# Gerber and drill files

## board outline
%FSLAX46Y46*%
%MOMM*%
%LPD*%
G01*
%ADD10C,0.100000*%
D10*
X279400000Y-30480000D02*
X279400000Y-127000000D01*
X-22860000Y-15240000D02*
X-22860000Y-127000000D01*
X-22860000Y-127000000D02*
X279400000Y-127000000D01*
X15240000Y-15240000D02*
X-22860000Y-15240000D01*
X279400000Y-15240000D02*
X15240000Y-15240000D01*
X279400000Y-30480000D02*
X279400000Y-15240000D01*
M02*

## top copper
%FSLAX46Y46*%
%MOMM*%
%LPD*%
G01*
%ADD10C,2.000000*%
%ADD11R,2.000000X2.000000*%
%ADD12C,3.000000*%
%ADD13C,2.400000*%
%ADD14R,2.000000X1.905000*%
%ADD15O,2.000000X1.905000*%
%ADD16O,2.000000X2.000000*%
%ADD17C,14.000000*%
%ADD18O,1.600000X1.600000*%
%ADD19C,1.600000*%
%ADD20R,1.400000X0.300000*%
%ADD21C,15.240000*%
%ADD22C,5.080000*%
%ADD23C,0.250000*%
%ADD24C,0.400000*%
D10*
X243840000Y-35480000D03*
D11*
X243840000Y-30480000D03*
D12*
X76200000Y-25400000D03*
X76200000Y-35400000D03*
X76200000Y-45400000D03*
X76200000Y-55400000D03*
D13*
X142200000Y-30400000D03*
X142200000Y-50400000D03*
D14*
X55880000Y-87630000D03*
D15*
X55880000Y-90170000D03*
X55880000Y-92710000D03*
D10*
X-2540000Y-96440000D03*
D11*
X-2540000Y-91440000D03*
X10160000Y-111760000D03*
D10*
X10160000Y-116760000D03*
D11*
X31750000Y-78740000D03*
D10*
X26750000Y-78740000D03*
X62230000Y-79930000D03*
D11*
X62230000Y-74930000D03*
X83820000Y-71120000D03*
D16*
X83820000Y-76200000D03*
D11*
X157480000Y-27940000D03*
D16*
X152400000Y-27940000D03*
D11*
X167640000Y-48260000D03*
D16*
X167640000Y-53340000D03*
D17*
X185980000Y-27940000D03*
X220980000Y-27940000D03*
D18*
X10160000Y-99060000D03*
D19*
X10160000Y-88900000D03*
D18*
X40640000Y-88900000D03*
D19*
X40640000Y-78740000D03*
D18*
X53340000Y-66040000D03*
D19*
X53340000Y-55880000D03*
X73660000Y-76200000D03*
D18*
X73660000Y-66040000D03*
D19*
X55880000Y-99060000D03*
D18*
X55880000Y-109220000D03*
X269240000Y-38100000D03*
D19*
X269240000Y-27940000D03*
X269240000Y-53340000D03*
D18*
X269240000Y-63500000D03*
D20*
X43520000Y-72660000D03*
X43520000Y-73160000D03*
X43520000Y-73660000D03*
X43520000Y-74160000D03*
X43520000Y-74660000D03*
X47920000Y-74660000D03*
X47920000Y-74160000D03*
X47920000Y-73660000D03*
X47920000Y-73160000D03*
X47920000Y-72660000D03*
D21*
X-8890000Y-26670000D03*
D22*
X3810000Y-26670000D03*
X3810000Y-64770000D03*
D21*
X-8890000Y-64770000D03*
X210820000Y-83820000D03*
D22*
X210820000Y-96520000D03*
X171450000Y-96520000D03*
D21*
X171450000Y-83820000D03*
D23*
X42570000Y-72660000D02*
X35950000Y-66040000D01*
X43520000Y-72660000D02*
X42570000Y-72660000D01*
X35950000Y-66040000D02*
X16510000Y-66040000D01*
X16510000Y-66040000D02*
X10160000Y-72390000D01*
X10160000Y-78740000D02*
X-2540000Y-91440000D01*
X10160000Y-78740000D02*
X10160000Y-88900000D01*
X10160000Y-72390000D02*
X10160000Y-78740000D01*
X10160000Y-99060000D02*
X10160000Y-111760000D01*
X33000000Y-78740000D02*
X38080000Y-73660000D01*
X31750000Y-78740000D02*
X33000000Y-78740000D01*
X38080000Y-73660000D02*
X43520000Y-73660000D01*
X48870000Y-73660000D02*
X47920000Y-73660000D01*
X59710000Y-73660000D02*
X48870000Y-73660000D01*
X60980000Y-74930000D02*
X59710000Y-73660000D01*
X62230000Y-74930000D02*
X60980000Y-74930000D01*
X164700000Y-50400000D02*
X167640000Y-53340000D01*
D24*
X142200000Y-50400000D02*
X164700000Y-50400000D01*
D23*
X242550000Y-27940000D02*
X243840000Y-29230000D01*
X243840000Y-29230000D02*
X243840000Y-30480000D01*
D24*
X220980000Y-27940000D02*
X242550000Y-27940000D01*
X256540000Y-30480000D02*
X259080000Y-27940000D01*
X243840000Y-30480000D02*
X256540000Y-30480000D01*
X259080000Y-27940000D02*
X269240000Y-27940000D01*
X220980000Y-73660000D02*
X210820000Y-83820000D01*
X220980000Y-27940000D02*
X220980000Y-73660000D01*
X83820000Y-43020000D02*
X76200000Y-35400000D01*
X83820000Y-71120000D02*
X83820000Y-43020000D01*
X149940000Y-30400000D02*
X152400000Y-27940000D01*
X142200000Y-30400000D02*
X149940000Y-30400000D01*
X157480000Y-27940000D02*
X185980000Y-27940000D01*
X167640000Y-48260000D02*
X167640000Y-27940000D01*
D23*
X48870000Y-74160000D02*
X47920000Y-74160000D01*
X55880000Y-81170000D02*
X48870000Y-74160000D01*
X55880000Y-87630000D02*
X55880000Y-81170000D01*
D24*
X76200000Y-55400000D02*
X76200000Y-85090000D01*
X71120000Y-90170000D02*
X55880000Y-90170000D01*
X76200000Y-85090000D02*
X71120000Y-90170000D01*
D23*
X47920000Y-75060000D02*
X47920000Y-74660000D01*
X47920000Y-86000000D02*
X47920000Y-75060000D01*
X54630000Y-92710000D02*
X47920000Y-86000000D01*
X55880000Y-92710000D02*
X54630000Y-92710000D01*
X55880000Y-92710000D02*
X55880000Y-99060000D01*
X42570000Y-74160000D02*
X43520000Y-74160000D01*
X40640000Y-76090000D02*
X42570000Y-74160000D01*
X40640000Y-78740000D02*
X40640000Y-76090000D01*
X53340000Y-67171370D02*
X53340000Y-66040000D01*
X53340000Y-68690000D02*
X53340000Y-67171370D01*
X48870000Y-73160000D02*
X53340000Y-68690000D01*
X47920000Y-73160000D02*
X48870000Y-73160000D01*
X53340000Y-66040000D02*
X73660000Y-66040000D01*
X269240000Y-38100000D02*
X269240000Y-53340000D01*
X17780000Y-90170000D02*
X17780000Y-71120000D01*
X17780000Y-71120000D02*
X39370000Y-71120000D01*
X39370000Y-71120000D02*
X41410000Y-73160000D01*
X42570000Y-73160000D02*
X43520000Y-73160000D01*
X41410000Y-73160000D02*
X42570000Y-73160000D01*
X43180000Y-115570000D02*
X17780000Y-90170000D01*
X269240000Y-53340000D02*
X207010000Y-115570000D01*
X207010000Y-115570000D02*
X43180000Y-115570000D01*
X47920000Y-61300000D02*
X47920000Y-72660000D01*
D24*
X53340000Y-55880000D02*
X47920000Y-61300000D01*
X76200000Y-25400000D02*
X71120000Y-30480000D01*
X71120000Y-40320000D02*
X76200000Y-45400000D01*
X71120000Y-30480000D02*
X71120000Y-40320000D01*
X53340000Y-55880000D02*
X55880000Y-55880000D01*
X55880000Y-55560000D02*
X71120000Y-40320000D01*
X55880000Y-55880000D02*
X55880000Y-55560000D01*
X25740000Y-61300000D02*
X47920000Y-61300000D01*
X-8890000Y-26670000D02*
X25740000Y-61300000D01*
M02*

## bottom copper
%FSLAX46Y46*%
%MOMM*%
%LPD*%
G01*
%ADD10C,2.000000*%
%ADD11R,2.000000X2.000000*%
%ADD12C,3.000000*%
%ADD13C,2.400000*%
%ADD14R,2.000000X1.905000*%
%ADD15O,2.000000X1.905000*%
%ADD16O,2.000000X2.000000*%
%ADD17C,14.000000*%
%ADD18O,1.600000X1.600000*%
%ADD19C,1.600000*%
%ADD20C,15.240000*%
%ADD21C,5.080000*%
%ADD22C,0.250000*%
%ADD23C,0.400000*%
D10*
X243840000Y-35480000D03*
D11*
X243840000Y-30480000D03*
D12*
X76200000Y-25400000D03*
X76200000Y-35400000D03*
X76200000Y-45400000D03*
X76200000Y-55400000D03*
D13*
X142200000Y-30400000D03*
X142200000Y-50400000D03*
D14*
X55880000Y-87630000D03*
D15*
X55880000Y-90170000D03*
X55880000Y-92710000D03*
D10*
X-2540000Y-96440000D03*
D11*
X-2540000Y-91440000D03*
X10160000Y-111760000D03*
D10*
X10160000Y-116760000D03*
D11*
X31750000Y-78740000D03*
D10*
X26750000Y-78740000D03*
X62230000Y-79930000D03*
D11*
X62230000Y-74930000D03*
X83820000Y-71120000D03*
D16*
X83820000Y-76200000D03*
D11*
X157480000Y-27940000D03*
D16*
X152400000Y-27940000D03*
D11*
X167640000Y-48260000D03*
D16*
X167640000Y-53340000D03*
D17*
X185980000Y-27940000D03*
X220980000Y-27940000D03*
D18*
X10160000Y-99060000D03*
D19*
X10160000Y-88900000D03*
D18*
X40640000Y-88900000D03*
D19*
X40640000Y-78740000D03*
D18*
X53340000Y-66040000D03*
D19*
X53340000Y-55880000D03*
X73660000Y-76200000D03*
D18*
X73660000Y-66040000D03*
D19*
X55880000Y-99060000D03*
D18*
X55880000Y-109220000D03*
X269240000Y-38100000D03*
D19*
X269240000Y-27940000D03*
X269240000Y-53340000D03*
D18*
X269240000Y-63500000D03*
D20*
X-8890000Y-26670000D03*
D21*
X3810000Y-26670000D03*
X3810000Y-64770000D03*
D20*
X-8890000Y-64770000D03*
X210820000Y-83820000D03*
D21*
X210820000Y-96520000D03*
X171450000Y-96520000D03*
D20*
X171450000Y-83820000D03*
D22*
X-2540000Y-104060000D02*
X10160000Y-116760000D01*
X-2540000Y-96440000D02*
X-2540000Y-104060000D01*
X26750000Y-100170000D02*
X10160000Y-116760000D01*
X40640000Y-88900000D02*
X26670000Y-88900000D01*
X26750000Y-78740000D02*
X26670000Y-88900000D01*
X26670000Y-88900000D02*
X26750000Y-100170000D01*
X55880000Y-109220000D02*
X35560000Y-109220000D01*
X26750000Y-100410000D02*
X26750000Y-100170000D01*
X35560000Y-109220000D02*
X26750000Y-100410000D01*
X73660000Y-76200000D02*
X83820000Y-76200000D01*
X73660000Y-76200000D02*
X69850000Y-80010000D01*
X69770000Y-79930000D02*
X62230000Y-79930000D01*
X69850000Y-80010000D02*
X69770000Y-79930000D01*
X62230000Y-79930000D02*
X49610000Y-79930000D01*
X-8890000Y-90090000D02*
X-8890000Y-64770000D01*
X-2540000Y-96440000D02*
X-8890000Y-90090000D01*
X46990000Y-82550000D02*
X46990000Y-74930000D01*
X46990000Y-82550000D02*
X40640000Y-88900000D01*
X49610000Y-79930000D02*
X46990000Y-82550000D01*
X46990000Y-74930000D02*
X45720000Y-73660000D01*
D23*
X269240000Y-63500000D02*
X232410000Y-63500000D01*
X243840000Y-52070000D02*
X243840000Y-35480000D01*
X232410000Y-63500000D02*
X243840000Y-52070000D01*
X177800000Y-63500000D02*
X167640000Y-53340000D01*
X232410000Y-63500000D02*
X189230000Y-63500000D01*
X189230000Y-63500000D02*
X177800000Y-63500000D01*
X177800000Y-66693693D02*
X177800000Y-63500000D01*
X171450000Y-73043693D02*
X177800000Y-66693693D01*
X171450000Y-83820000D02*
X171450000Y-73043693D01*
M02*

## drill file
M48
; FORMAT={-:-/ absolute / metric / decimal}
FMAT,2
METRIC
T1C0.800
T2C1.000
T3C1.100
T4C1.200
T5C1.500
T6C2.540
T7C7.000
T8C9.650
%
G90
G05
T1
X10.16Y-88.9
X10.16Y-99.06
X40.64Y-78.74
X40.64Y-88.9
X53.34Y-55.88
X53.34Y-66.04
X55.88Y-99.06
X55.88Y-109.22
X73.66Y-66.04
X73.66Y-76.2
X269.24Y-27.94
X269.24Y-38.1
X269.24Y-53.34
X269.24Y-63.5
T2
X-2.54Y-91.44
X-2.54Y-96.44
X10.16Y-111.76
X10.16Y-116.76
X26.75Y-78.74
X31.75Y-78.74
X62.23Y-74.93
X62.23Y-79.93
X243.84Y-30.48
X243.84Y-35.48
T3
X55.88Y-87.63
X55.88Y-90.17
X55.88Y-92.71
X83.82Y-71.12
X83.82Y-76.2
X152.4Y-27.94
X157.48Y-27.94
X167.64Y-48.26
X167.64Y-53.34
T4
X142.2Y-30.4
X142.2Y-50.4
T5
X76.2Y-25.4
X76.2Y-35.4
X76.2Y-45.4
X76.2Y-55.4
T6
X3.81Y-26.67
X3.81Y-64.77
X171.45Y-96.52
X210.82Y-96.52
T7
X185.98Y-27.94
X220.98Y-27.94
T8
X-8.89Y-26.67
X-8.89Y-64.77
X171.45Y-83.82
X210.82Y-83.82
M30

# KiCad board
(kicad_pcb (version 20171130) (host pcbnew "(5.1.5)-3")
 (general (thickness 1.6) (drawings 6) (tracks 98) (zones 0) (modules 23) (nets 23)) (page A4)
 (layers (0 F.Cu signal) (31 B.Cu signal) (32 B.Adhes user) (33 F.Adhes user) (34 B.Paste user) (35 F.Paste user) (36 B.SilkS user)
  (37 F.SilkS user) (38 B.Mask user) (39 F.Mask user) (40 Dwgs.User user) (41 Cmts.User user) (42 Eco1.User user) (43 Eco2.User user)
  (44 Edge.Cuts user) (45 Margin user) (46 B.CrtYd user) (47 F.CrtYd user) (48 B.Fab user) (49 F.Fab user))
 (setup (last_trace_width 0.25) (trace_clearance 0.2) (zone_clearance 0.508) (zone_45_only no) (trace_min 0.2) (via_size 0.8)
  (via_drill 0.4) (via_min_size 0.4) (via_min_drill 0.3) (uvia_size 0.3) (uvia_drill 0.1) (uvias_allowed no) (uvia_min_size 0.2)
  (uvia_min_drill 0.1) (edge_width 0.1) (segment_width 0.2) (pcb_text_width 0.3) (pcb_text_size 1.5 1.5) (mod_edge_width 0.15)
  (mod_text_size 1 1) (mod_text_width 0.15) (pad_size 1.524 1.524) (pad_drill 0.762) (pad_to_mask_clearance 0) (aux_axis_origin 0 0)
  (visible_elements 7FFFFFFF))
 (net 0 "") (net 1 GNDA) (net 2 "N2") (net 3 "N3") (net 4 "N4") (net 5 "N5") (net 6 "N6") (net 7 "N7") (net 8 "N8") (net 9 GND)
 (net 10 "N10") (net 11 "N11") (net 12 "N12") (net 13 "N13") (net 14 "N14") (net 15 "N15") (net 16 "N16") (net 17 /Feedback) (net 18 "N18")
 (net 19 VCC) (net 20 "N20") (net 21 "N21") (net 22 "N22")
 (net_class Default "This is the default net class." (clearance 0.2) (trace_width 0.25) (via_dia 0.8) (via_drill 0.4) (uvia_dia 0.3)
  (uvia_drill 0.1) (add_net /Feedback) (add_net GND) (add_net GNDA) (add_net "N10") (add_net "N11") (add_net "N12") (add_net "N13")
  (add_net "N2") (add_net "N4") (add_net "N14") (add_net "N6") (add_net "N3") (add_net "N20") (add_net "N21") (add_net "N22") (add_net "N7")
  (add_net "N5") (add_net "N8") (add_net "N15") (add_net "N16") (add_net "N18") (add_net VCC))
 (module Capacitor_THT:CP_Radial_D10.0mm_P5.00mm (layer F.Cu) (at 243.84 30.48 270)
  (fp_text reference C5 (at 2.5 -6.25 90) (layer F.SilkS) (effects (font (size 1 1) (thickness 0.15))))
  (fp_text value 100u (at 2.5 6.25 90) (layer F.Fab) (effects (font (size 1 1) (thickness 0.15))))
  (pad 2 thru_hole circle (at 5 0 270) (size 2 2) (drill 1) (layers *.Cu *.Mask) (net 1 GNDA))
  (pad 1 thru_hole rect (at 0 0 270) (size 2 2) (drill 1) (layers *.Cu *.Mask) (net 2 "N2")))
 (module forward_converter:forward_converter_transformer (layer F.Cu) (at 109.2 40.4)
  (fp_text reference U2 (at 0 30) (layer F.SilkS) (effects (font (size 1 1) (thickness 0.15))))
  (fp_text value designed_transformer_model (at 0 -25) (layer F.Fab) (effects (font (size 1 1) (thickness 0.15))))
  (pad 1 thru_hole circle (at -33 -15) (size 3 3) (drill 1.5) (layers *.Cu *.Mask) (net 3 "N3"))
  (pad 2 thru_hole circle (at -33 -5) (size 3 3) (drill 1.5) (layers *.Cu *.Mask) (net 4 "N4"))
  (pad 3 thru_hole circle (at -33 5) (size 3 3) (drill 1.5) (layers *.Cu *.Mask) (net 3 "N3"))
  (pad 4 thru_hole circle (at -33 15) (size 3 3) (drill 1.5) (layers *.Cu *.Mask) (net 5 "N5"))
  (pad 5 thru_hole circle (at 33 -10) (size 2.4 2.4) (drill 1.2) (layers *.Cu *.Mask) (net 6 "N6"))
  (pad 6 thru_hole circle (at 33 10) (size 2.4 2.4) (drill 1.2) (layers *.Cu *.Mask) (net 1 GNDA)))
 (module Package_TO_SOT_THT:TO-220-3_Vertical (layer F.Cu) (at 55.88 87.63 270)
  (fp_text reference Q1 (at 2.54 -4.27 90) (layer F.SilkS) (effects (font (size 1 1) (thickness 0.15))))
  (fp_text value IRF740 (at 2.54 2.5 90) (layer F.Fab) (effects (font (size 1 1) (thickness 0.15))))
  (pad 1 thru_hole rect (at 0 0 270) (size 1.905 2) (drill 1.1) (layers *.Cu *.Mask) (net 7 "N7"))
  (pad 2 thru_hole oval (at 2.54 0 270) (size 1.905 2) (drill 1.1) (layers *.Cu *.Mask) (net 5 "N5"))
  (pad 3 thru_hole oval (at 5.08 0 270) (size 1.905 2) (drill 1.1) (layers *.Cu *.Mask) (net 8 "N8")))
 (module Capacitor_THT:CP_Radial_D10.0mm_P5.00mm (layer F.Cu) (at -2.54 91.44 270)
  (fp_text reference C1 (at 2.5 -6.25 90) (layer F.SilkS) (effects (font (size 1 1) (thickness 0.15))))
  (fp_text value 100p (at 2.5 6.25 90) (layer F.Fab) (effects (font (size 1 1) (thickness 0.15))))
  (pad 2 thru_hole circle (at 5 0 270) (size 2 2) (drill 1) (layers *.Cu *.Mask) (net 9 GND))
  (pad 1 thru_hole rect (at 0 0 270) (size 2 2) (drill 1) (layers *.Cu *.Mask) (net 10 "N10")))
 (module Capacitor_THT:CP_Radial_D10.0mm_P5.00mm (layer F.Cu) (at 10.16 111.76 270)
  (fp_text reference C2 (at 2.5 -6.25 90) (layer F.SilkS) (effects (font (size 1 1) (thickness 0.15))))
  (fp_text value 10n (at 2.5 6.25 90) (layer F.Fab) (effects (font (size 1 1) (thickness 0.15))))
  (pad 1 thru_hole rect (at 0 0 270) (size 2 2) (drill 1) (layers *.Cu *.Mask) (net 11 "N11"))
  (pad 2 thru_hole circle (at 5 0 270) (size 2 2) (drill 1) (layers *.Cu *.Mask) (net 9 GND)))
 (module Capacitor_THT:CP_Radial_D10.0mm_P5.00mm (layer F.Cu) (at 31.75 78.74 180)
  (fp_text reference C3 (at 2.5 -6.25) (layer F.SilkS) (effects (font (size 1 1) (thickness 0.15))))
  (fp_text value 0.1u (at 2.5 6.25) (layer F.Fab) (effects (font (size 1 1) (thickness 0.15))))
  (pad 1 thru_hole rect (at 0 0 180) (size 2 2) (drill 1) (layers *.Cu *.Mask) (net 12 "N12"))
  (pad 2 thru_hole circle (at 5 0 180) (size 2 2) (drill 1) (layers *.Cu *.Mask) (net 9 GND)))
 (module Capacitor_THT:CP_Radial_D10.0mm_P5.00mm (layer F.Cu) (at 62.23 74.93 270)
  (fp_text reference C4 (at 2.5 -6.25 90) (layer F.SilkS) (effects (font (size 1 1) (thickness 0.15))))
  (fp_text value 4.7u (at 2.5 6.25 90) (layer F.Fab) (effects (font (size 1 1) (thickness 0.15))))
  (pad 2 thru_hole circle (at 5 0 270) (size 2 2) (drill 1) (layers *.Cu *.Mask) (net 9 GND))
  (pad 1 thru_hole rect (at 0 0 270) (size 2 2) (drill 1) (layers *.Cu *.Mask) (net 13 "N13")))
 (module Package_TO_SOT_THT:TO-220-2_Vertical (layer F.Cu) (at 83.82 71.12 270)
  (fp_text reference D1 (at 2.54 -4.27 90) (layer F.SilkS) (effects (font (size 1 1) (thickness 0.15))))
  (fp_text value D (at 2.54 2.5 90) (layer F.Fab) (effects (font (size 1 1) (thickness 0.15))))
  (pad 1 thru_hole rect (at 0 0 270) (size 2 2) (drill 1.1) (layers *.Cu *.Mask) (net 4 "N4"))
  (pad 2 thru_hole oval (at 5.08 0 270) (size 2 2) (drill 1.1) (layers *.Cu *.Mask) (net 9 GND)))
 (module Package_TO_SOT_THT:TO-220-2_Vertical (layer F.Cu) (at 157.48 27.94 180)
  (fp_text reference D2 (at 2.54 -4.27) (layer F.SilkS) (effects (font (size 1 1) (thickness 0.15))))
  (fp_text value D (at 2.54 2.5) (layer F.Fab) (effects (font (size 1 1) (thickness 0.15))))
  (pad 1 thru_hole rect (at 0 0 180) (size 2 2) (drill 1.1) (layers *.Cu *.Mask) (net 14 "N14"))
  (pad 2 thru_hole oval (at 5.08 0 180) (size 2 2) (drill 1.1) (layers *.Cu *.Mask) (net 6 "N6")))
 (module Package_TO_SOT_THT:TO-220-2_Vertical (layer F.Cu) (at 167.64 48.26 270)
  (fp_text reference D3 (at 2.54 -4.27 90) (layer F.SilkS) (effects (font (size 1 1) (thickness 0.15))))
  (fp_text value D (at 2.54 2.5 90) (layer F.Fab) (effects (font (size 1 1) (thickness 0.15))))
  (pad 1 thru_hole rect (at 0 0 270) (size 2 2) (drill 1.1) (layers *.Cu *.Mask) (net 14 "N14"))
  (pad 2 thru_hole oval (at 5.08 0 270) (size 2 2) (drill 1.1) (layers *.Cu *.Mask) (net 1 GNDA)))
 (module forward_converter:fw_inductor (layer F.Cu) (at 203.48 27.94 90)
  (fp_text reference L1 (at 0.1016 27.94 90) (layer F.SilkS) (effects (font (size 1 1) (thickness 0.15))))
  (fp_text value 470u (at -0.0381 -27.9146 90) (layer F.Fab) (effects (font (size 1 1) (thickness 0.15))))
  (pad 1 thru_hole circle (at 0 -17.5 90) (size 14 14) (drill 7) (layers *.Cu *.Mask) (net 14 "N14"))
  (pad 2 thru_hole circle (at 0 17.5 90) (size 14 14) (drill 7) (layers *.Cu *.Mask) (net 2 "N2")))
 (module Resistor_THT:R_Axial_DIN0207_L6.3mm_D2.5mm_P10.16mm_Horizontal (layer F.Cu) (at 10.16 88.9 270)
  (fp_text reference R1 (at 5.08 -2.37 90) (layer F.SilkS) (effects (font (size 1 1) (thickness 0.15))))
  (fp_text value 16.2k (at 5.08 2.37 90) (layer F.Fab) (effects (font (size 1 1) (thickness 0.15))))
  (pad 2 thru_hole oval (at 10.16 0 270) (size 1.6 1.6) (drill 0.8) (layers *.Cu *.Mask) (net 11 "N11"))
  (pad 1 thru_hole circle (at 0 0 270) (size 1.6 1.6) (drill 0.8) (layers *.Cu *.Mask) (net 10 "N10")))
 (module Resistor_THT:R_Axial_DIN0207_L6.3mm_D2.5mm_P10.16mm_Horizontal (layer F.Cu) (at 40.64 78.74 270)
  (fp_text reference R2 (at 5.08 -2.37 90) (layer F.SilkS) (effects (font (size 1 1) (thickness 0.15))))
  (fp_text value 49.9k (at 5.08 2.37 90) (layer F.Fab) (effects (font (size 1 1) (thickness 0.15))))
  (pad 2 thru_hole oval (at 10.16 0 270) (size 1.6 1.6) (drill 0.8) (layers *.Cu *.Mask) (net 9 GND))
  (pad 1 thru_hole circle (at 0 0 270) (size 1.6 1.6) (drill 0.8) (layers *.Cu *.Mask) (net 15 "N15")))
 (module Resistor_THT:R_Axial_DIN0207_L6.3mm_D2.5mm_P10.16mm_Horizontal (layer F.Cu) (at 53.34 55.88 270)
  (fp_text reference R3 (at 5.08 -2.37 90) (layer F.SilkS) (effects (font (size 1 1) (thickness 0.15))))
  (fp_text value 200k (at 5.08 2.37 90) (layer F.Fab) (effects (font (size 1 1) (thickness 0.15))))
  (pad 2 thru_hole oval (at 10.16 0 270) (size 1.6 1.6) (drill 0.8) (layers *.Cu *.Mask) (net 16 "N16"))
  (pad 1 thru_hole circle (at 0 0 270) (size 1.6 1.6) (drill 0.8) (layers *.Cu *.Mask) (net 3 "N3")))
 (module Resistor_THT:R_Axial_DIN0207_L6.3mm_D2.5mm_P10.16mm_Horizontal (layer F.Cu) (at 73.66 76.2 90)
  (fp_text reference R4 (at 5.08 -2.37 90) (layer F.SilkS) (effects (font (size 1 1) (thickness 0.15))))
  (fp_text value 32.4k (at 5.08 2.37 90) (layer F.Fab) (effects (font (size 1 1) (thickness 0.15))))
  (pad 1 thru_hole circle (at 0 0 90) (size 1.6 1.6) (drill 0.8) (layers *.Cu *.Mask) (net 9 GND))
  (pad 2 thru_hole oval (at 10.16 0 90) (size 1.6 1.6) (drill 0.8) (layers *.Cu *.Mask) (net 16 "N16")))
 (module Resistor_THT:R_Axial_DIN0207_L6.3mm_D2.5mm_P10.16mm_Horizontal (layer F.Cu) (at 55.88 99.06 270)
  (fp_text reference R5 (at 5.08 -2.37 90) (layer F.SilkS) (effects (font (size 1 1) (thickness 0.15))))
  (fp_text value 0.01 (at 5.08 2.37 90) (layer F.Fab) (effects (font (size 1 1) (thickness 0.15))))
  (pad 1 thru_hole circle (at 0 0 270) (size 1.6 1.6) (drill 0.8) (layers *.Cu *.Mask) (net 8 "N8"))
  (pad 2 thru_hole oval (at 10.16 0 270) (size 1.6 1.6) (drill 0.8) (layers *.Cu *.Mask) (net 9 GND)))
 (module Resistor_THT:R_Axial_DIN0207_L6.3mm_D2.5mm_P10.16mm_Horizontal (layer F.Cu) (at 269.24 27.94 270)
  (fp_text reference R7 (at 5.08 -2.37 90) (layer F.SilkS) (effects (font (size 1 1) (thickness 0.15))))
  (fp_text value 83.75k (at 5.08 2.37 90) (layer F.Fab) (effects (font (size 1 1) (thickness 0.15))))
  (pad 2 thru_hole oval (at 10.16 0 270) (size 1.6 1.6) (drill 0.8) (layers *.Cu *.Mask) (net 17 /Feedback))
  (pad 1 thru_hole circle (at 0 0 270) (size 1.6 1.6) (drill 0.8) (layers *.Cu *.Mask) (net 2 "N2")))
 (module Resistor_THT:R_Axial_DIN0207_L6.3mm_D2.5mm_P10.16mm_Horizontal (layer F.Cu) (at 269.24 53.34 270)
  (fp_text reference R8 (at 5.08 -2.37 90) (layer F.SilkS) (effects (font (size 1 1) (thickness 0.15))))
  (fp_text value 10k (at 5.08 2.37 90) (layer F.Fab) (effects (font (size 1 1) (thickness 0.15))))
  (pad 1 thru_hole circle (at 0 0 270) (size 1.6 1.6) (drill 0.8) (layers *.Cu *.Mask) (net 17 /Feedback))
  (pad 2 thru_hole oval (at 10.16 0 270) (size 1.6 1.6) (drill 0.8) (layers *.Cu *.Mask) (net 1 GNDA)))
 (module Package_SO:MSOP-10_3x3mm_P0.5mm (layer F.Cu) (at 45.72 73.66)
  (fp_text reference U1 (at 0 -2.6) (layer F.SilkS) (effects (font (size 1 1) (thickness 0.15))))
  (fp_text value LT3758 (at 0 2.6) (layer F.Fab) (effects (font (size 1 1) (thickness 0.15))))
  (pad 1 smd rect (at -2.2 -1) (size 1.4 0.3) (layers F.Cu F.Paste F.Mask) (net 10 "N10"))
  (pad 2 smd rect (at -2.2 -0.5) (size 1.4 0.3) (layers F.Cu F.Paste F.Mask) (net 17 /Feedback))
  (pad 3 smd rect (at -2.2 0) (size 1.4 0.3) (layers F.Cu F.Paste F.Mask) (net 12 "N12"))
  (pad 4 smd rect (at -2.2 0.5) (size 1.4 0.3) (layers F.Cu F.Paste F.Mask) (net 15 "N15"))
  (pad 5 smd rect (at -2.2 1) (size 1.4 0.3) (layers F.Cu F.Paste F.Mask) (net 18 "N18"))
  (pad 6 smd rect (at 2.2 1) (size 1.4 0.3) (layers F.Cu F.Paste F.Mask) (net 8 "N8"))
  (pad 7 smd rect (at 2.2 0.5) (size 1.4 0.3) (layers F.Cu F.Paste F.Mask) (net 7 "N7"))
  (pad 8 smd rect (at 2.2 0) (size 1.4 0.3) (layers F.Cu F.Paste F.Mask) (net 13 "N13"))
  (pad 9 smd rect (at 2.2 -0.5) (size 1.4 0.3) (layers F.Cu F.Paste F.Mask) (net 16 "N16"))
  (pad 10 smd rect (at 2.2 -1) (size 1.4 0.3) (layers F.Cu F.Paste F.Mask) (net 3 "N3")))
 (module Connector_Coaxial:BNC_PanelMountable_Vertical (layer F.Cu) (at 3.81 26.67)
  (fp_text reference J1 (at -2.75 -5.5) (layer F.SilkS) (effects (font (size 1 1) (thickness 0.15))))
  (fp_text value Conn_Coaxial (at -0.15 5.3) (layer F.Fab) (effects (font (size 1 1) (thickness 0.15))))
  (pad 2 thru_hole circle (at -12.7 0) (size 15.24 15.24) (drill 9.65) (layers *.Cu *.Mask) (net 3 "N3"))
  (pad 1 thru_hole circle (at 0 0) (size 5.08 5.08) (drill 2.54) (layers *.Cu *.Mask) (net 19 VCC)))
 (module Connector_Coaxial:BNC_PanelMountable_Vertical (layer F.Cu) (at 3.81 64.77)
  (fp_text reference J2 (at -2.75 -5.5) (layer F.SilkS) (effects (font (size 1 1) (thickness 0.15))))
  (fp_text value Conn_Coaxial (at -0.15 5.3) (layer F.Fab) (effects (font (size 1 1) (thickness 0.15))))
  (pad 1 thru_hole circle (at 0 0) (size 5.08 5.08) (drill 2.54) (layers *.Cu *.Mask) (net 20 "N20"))
  (pad 2 thru_hole circle (at -12.7 0) (size 15.24 15.24) (drill 9.65) (layers *.Cu *.Mask) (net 9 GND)))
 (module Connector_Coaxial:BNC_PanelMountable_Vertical (layer F.Cu) (at 210.82 96.52 270)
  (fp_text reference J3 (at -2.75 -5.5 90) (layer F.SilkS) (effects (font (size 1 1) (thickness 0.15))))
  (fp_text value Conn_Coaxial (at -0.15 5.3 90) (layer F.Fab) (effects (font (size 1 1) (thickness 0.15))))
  (pad 2 thru_hole circle (at -12.7 0 270) (size 15.24 15.24) (drill 9.65) (layers *.Cu *.Mask) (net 2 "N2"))
  (pad 1 thru_hole circle (at 0 0 270) (size 5.08 5.08) (drill 2.54) (layers *.Cu *.Mask) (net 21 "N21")))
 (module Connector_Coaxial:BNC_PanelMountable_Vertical (layer F.Cu) (at 171.45 96.52 270)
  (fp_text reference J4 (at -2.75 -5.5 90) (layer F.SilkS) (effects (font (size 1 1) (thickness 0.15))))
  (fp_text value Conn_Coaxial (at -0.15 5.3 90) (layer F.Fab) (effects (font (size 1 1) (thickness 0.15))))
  (pad 1 thru_hole circle (at 0 0 270) (size 5.08 5.08) (drill 2.54) (layers *.Cu *.Mask) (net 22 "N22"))
  (pad 2 thru_hole circle (at -12.7 0 270) (size 15.24 15.24) (drill 9.65) (layers *.Cu *.Mask) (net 1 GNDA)))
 (gr_line (start 279.4 30.48) (end 279.4 127) (layer Edge.Cuts) (width 0.1))
 (gr_line (start -22.86 15.24) (end -22.86 127) (layer Edge.Cuts) (width 0.1))
 (gr_line (start -22.86 127) (end 279.4 127) (layer Edge.Cuts) (width 0.1))
 (gr_line (start 15.24 15.24) (end -22.86 15.24) (layer Edge.Cuts) (width 0.1))
 (gr_line (start 279.4 15.24) (end 15.24 15.24) (layer Edge.Cuts) (width 0.1))
 (gr_line (start 279.4 30.48) (end 279.4 15.24) (layer Edge.Cuts) (width 0.1))
 (segment (start -2.54 104.06) (end 10.16 116.76) (width 0.25) (layer B.Cu) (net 9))
 (segment (start -2.54 96.44) (end -2.54 104.06) (width 0.25) (layer B.Cu) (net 9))
 (segment (start 26.75 100.17) (end 10.16 116.76) (width 0.25) (layer B.Cu) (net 9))
 (segment (start 40.64 88.9) (end 26.67 88.9) (width 0.25) (layer B.Cu) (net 9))
 (segment (start 26.75 78.74) (end 26.67 88.9) (width 0.25) (layer B.Cu) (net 9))
 (segment (start 26.67 88.9) (end 26.75 100.17) (width 0.25) (layer B.Cu) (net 9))
 (segment (start 55.88 109.22) (end 35.56 109.22) (width 0.25) (layer B.Cu) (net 9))
 (segment (start 26.75 100.41) (end 26.75 100.17) (width 0.25) (layer B.Cu) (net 9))
 (segment (start 35.56 109.22) (end 26.75 100.41) (width 0.25) (layer B.Cu) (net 9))
 (segment (start 73.66 76.2) (end 83.82 76.2) (width 0.25) (layer B.Cu) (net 9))
 (segment (start 73.66 76.2) (end 69.85 80.01) (width 0.25) (layer B.Cu) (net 9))
 (segment (start 69.77 79.93) (end 62.23 79.93) (width 0.25) (layer B.Cu) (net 9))
 (segment (start 69.85 80.01) (end 69.77 79.93) (width 0.25) (layer B.Cu) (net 9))
 (segment (start 62.23 79.93) (end 49.61 79.93) (width 0.25) (layer B.Cu) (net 9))
 (segment (start -8.89 90.09) (end -8.89 64.77) (width 0.25) (layer B.Cu) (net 9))
 (segment (start -2.54 96.44) (end -8.89 90.09) (width 0.25) (layer B.Cu) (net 9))
 (segment (start 46.99 82.55) (end 46.99 74.93) (width 0.25) (layer B.Cu) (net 9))
 (segment (start 46.99 82.55) (end 40.64 88.9) (width 0.25) (layer B.Cu) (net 9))
 (segment (start 49.61 79.93) (end 46.99 82.55) (width 0.25) (layer B.Cu) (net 9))
 (segment (start 46.99 74.93) (end 45.72 73.66) (width 0.25) (layer B.Cu) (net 9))
 (segment (start 42.57 72.66) (end 35.95 66.04) (width 0.25) (layer F.Cu) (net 10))
 (segment (start 43.52 72.66) (end 42.57 72.66) (width 0.25) (layer F.Cu) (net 10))
 (segment (start 35.95 66.04) (end 16.51 66.04) (width 0.25) (layer F.Cu) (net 10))
 (segment (start 16.51 66.04) (end 10.16 72.39) (width 0.25) (layer F.Cu) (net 10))
 (segment (start 10.16 78.74) (end -2.54 91.44) (width 0.25) (layer F.Cu) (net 10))
 (segment (start 10.16 78.74) (end 10.16 88.9) (width 0.25) (layer F.Cu) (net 10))
 (segment (start 10.16 72.39) (end 10.16 78.74) (width 0.25) (layer F.Cu) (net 10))
 (segment (start 10.16 99.06) (end 10.16 111.76) (width 0.25) (layer F.Cu) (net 11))
 (segment (start 33 78.74) (end 38.08 73.66) (width 0.25) (layer F.Cu) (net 12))
 (segment (start 31.75 78.74) (end 33 78.74) (width 0.25) (layer F.Cu) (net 12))
 (segment (start 38.08 73.66) (end 43.52 73.66) (width 0.25) (layer F.Cu) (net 12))
 (segment (start 48.87 73.66) (end 47.92 73.66) (width 0.25) (layer F.Cu) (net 13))
 (segment (start 59.71 73.66) (end 48.87 73.66) (width 0.25) (layer F.Cu) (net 13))
 (segment (start 60.98 74.93) (end 59.71 73.66) (width 0.25) (layer F.Cu) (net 13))
 (segment (start 62.23 74.93) (end 60.98 74.93) (width 0.25) (layer F.Cu) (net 13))
 (segment (start 164.7 50.4) (end 167.64 53.34) (width 0.25) (layer F.Cu) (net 1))
 (segment (start 142.2 50.4) (end 164.7 50.4) (width 0.4) (layer F.Cu) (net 1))
 (segment (start 269.24 63.5) (end 232.41 63.5) (width 0.4) (layer B.Cu) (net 1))
 (segment (start 243.84 52.07) (end 243.84 35.48) (width 0.4) (layer B.Cu) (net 1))
 (segment (start 232.41 63.5) (end 243.84 52.07) (width 0.4) (layer B.Cu) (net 1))
 (segment (start 177.8 63.5) (end 167.64 53.34) (width 0.4) (layer B.Cu) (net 1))
 (segment (start 232.41 63.5) (end 189.23 63.5) (width 0.4) (layer B.Cu) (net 1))
 (segment (start 189.23 63.5) (end 177.8 63.5) (width 0.4) (layer B.Cu) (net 1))
 (segment (start 177.8 66.693693) (end 177.8 63.5) (width 0.4) (layer B.Cu) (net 1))
 (segment (start 171.45 73.043693) (end 177.8 66.693693) (width 0.4) (layer B.Cu) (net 1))
 (segment (start 171.45 83.82) (end 171.45 73.043693) (width 0.4) (layer B.Cu) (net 1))
 (segment (start 242.55 27.94) (end 243.84 29.23) (width 0.25) (layer F.Cu) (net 2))
 (segment (start 243.84 29.23) (end 243.84 30.48) (width 0.25) (layer F.Cu) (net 2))
 (segment (start 220.98 27.94) (end 242.55 27.94) (width 0.4) (layer F.Cu) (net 2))
 (segment (start 256.54 30.48) (end 259.08 27.94) (width 0.4) (layer F.Cu) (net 2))
 (segment (start 243.84 30.48) (end 256.54 30.48) (width 0.4) (layer F.Cu) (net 2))
 (segment (start 259.08 27.94) (end 269.24 27.94) (width 0.4) (layer F.Cu) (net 2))
 (segment (start 220.98 73.66) (end 210.82 83.82) (width 0.4) (layer F.Cu) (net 2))
 (segment (start 220.98 27.94) (end 220.98 73.66) (width 0.4) (layer F.Cu) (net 2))
 (segment (start 83.82 43.02) (end 76.2 35.4) (width 0.4) (layer F.Cu) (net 4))
 (segment (start 83.82 71.12) (end 83.82 43.02) (width 0.4) (layer F.Cu) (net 4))
 (segment (start 149.94 30.4) (end 152.4 27.94) (width 0.4) (layer F.Cu) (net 6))
 (segment (start 142.2 30.4) (end 149.94 30.4) (width 0.4) (layer F.Cu) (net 6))
 (segment (start 157.48 27.94) (end 185.98 27.94) (width 0.4) (layer F.Cu) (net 14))
 (segment (start 167.64 48.26) (end 167.64 27.94) (width 0.4) (layer F.Cu) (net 14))
 (segment (start 48.87 74.16) (end 47.92 74.16) (width 0.25) (layer F.Cu) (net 7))
 (segment (start 55.88 81.17) (end 48.87 74.16) (width 0.25) (layer F.Cu) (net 7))
 (segment (start 55.88 87.63) (end 55.88 81.17) (width 0.25) (layer F.Cu) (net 7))
 (segment (start 76.2 55.4) (end 76.2 85.09) (width 0.4) (layer F.Cu) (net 5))
 (segment (start 71.12 90.17) (end 55.88 90.17) (width 0.4) (layer F.Cu) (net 5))
 (segment (start 76.2 85.09) (end 71.12 90.17) (width 0.4) (layer F.Cu) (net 5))
 (segment (start 47.92 75.06) (end 47.92 74.66) (width 0.25) (layer F.Cu) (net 8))
 (segment (start 47.92 86) (end 47.92 75.06) (width 0.25) (layer F.Cu) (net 8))
 (segment (start 54.63 92.71) (end 47.92 86) (width 0.25) (layer F.Cu) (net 8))
 (segment (start 55.88 92.71) (end 54.63 92.71) (width 0.25) (layer F.Cu) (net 8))
 (segment (start 55.88 92.71) (end 55.88 99.06) (width 0.25) (layer F.Cu) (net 8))
 (segment (start 42.57 74.16) (end 43.52 74.16) (width 0.25) (layer F.Cu) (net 15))
 (segment (start 40.64 76.09) (end 42.57 74.16) (width 0.25) (layer F.Cu) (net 15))
 (segment (start 40.64 78.74) (end 40.64 76.09) (width 0.25) (layer F.Cu) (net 15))
 (segment (start 53.34 67.17137) (end 53.34 66.04) (width 0.25) (layer F.Cu) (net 16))
 (segment (start 53.34 68.69) (end 53.34 67.17137) (width 0.25) (layer F.Cu) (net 16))
 (segment (start 48.87 73.16) (end 53.34 68.69) (width 0.25) (layer F.Cu) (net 16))
 (segment (start 47.92 73.16) (end 48.87 73.16) (width 0.25) (layer F.Cu) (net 16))
 (segment (start 53.34 66.04) (end 73.66 66.04) (width 0.25) (layer F.Cu) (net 16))
 (segment (start 269.24 38.1) (end 269.24 53.34) (width 0.25) (layer F.Cu) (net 17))
 (segment (start 17.78 90.17) (end 17.78 71.12) (width 0.25) (layer F.Cu) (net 17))
 (segment (start 17.78 71.12) (end 39.37 71.12) (width 0.25) (layer F.Cu) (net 17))
 (segment (start 39.37 71.12) (end 41.41 73.16) (width 0.25) (layer F.Cu) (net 17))
 (segment (start 42.57 73.16) (end 43.52 73.16) (width 0.25) (layer F.Cu) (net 17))
 (segment (start 41.41 73.16) (end 42.57 73.16) (width 0.25) (layer F.Cu) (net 17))
 (segment (start 43.18 115.57) (end 17.78 90.17) (width 0.25) (layer F.Cu) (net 17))
 (segment (start 269.24 53.34) (end 207.01 115.57) (width 0.25) (layer F.Cu) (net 17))
 (segment (start 207.01 115.57) (end 43.18 115.57) (width 0.25) (layer F.Cu) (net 17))
 (segment (start 47.92 61.3) (end 47.92 72.66) (width 0.25) (layer F.Cu) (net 3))
 (segment (start 53.34 55.88) (end 47.92 61.3) (width 0.4) (layer F.Cu) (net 3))
 (segment (start 76.2 25.4) (end 71.12 30.48) (width 0.4) (layer F.Cu) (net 3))
 (segment (start 71.12 40.32) (end 76.2 45.4) (width 0.4) (layer F.Cu) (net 3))
 (segment (start 71.12 30.48) (end 71.12 40.32) (width 0.4) (layer F.Cu) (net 3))
 (segment (start 53.34 55.88) (end 55.88 55.88) (width 0.4) (layer F.Cu) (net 3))
 (segment (start 55.88 55.56) (end 71.12 40.32) (width 0.4) (layer F.Cu) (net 3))
 (segment (start 55.88 55.88) (end 55.88 55.56) (width 0.4) (layer F.Cu) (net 3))
 (segment (start 25.74 61.3) (end 47.92 61.3) (width 0.4) (layer F.Cu) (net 3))
 (segment (start -8.89 26.67) (end 25.74 61.3) (width 0.4) (layer F.Cu) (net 3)))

